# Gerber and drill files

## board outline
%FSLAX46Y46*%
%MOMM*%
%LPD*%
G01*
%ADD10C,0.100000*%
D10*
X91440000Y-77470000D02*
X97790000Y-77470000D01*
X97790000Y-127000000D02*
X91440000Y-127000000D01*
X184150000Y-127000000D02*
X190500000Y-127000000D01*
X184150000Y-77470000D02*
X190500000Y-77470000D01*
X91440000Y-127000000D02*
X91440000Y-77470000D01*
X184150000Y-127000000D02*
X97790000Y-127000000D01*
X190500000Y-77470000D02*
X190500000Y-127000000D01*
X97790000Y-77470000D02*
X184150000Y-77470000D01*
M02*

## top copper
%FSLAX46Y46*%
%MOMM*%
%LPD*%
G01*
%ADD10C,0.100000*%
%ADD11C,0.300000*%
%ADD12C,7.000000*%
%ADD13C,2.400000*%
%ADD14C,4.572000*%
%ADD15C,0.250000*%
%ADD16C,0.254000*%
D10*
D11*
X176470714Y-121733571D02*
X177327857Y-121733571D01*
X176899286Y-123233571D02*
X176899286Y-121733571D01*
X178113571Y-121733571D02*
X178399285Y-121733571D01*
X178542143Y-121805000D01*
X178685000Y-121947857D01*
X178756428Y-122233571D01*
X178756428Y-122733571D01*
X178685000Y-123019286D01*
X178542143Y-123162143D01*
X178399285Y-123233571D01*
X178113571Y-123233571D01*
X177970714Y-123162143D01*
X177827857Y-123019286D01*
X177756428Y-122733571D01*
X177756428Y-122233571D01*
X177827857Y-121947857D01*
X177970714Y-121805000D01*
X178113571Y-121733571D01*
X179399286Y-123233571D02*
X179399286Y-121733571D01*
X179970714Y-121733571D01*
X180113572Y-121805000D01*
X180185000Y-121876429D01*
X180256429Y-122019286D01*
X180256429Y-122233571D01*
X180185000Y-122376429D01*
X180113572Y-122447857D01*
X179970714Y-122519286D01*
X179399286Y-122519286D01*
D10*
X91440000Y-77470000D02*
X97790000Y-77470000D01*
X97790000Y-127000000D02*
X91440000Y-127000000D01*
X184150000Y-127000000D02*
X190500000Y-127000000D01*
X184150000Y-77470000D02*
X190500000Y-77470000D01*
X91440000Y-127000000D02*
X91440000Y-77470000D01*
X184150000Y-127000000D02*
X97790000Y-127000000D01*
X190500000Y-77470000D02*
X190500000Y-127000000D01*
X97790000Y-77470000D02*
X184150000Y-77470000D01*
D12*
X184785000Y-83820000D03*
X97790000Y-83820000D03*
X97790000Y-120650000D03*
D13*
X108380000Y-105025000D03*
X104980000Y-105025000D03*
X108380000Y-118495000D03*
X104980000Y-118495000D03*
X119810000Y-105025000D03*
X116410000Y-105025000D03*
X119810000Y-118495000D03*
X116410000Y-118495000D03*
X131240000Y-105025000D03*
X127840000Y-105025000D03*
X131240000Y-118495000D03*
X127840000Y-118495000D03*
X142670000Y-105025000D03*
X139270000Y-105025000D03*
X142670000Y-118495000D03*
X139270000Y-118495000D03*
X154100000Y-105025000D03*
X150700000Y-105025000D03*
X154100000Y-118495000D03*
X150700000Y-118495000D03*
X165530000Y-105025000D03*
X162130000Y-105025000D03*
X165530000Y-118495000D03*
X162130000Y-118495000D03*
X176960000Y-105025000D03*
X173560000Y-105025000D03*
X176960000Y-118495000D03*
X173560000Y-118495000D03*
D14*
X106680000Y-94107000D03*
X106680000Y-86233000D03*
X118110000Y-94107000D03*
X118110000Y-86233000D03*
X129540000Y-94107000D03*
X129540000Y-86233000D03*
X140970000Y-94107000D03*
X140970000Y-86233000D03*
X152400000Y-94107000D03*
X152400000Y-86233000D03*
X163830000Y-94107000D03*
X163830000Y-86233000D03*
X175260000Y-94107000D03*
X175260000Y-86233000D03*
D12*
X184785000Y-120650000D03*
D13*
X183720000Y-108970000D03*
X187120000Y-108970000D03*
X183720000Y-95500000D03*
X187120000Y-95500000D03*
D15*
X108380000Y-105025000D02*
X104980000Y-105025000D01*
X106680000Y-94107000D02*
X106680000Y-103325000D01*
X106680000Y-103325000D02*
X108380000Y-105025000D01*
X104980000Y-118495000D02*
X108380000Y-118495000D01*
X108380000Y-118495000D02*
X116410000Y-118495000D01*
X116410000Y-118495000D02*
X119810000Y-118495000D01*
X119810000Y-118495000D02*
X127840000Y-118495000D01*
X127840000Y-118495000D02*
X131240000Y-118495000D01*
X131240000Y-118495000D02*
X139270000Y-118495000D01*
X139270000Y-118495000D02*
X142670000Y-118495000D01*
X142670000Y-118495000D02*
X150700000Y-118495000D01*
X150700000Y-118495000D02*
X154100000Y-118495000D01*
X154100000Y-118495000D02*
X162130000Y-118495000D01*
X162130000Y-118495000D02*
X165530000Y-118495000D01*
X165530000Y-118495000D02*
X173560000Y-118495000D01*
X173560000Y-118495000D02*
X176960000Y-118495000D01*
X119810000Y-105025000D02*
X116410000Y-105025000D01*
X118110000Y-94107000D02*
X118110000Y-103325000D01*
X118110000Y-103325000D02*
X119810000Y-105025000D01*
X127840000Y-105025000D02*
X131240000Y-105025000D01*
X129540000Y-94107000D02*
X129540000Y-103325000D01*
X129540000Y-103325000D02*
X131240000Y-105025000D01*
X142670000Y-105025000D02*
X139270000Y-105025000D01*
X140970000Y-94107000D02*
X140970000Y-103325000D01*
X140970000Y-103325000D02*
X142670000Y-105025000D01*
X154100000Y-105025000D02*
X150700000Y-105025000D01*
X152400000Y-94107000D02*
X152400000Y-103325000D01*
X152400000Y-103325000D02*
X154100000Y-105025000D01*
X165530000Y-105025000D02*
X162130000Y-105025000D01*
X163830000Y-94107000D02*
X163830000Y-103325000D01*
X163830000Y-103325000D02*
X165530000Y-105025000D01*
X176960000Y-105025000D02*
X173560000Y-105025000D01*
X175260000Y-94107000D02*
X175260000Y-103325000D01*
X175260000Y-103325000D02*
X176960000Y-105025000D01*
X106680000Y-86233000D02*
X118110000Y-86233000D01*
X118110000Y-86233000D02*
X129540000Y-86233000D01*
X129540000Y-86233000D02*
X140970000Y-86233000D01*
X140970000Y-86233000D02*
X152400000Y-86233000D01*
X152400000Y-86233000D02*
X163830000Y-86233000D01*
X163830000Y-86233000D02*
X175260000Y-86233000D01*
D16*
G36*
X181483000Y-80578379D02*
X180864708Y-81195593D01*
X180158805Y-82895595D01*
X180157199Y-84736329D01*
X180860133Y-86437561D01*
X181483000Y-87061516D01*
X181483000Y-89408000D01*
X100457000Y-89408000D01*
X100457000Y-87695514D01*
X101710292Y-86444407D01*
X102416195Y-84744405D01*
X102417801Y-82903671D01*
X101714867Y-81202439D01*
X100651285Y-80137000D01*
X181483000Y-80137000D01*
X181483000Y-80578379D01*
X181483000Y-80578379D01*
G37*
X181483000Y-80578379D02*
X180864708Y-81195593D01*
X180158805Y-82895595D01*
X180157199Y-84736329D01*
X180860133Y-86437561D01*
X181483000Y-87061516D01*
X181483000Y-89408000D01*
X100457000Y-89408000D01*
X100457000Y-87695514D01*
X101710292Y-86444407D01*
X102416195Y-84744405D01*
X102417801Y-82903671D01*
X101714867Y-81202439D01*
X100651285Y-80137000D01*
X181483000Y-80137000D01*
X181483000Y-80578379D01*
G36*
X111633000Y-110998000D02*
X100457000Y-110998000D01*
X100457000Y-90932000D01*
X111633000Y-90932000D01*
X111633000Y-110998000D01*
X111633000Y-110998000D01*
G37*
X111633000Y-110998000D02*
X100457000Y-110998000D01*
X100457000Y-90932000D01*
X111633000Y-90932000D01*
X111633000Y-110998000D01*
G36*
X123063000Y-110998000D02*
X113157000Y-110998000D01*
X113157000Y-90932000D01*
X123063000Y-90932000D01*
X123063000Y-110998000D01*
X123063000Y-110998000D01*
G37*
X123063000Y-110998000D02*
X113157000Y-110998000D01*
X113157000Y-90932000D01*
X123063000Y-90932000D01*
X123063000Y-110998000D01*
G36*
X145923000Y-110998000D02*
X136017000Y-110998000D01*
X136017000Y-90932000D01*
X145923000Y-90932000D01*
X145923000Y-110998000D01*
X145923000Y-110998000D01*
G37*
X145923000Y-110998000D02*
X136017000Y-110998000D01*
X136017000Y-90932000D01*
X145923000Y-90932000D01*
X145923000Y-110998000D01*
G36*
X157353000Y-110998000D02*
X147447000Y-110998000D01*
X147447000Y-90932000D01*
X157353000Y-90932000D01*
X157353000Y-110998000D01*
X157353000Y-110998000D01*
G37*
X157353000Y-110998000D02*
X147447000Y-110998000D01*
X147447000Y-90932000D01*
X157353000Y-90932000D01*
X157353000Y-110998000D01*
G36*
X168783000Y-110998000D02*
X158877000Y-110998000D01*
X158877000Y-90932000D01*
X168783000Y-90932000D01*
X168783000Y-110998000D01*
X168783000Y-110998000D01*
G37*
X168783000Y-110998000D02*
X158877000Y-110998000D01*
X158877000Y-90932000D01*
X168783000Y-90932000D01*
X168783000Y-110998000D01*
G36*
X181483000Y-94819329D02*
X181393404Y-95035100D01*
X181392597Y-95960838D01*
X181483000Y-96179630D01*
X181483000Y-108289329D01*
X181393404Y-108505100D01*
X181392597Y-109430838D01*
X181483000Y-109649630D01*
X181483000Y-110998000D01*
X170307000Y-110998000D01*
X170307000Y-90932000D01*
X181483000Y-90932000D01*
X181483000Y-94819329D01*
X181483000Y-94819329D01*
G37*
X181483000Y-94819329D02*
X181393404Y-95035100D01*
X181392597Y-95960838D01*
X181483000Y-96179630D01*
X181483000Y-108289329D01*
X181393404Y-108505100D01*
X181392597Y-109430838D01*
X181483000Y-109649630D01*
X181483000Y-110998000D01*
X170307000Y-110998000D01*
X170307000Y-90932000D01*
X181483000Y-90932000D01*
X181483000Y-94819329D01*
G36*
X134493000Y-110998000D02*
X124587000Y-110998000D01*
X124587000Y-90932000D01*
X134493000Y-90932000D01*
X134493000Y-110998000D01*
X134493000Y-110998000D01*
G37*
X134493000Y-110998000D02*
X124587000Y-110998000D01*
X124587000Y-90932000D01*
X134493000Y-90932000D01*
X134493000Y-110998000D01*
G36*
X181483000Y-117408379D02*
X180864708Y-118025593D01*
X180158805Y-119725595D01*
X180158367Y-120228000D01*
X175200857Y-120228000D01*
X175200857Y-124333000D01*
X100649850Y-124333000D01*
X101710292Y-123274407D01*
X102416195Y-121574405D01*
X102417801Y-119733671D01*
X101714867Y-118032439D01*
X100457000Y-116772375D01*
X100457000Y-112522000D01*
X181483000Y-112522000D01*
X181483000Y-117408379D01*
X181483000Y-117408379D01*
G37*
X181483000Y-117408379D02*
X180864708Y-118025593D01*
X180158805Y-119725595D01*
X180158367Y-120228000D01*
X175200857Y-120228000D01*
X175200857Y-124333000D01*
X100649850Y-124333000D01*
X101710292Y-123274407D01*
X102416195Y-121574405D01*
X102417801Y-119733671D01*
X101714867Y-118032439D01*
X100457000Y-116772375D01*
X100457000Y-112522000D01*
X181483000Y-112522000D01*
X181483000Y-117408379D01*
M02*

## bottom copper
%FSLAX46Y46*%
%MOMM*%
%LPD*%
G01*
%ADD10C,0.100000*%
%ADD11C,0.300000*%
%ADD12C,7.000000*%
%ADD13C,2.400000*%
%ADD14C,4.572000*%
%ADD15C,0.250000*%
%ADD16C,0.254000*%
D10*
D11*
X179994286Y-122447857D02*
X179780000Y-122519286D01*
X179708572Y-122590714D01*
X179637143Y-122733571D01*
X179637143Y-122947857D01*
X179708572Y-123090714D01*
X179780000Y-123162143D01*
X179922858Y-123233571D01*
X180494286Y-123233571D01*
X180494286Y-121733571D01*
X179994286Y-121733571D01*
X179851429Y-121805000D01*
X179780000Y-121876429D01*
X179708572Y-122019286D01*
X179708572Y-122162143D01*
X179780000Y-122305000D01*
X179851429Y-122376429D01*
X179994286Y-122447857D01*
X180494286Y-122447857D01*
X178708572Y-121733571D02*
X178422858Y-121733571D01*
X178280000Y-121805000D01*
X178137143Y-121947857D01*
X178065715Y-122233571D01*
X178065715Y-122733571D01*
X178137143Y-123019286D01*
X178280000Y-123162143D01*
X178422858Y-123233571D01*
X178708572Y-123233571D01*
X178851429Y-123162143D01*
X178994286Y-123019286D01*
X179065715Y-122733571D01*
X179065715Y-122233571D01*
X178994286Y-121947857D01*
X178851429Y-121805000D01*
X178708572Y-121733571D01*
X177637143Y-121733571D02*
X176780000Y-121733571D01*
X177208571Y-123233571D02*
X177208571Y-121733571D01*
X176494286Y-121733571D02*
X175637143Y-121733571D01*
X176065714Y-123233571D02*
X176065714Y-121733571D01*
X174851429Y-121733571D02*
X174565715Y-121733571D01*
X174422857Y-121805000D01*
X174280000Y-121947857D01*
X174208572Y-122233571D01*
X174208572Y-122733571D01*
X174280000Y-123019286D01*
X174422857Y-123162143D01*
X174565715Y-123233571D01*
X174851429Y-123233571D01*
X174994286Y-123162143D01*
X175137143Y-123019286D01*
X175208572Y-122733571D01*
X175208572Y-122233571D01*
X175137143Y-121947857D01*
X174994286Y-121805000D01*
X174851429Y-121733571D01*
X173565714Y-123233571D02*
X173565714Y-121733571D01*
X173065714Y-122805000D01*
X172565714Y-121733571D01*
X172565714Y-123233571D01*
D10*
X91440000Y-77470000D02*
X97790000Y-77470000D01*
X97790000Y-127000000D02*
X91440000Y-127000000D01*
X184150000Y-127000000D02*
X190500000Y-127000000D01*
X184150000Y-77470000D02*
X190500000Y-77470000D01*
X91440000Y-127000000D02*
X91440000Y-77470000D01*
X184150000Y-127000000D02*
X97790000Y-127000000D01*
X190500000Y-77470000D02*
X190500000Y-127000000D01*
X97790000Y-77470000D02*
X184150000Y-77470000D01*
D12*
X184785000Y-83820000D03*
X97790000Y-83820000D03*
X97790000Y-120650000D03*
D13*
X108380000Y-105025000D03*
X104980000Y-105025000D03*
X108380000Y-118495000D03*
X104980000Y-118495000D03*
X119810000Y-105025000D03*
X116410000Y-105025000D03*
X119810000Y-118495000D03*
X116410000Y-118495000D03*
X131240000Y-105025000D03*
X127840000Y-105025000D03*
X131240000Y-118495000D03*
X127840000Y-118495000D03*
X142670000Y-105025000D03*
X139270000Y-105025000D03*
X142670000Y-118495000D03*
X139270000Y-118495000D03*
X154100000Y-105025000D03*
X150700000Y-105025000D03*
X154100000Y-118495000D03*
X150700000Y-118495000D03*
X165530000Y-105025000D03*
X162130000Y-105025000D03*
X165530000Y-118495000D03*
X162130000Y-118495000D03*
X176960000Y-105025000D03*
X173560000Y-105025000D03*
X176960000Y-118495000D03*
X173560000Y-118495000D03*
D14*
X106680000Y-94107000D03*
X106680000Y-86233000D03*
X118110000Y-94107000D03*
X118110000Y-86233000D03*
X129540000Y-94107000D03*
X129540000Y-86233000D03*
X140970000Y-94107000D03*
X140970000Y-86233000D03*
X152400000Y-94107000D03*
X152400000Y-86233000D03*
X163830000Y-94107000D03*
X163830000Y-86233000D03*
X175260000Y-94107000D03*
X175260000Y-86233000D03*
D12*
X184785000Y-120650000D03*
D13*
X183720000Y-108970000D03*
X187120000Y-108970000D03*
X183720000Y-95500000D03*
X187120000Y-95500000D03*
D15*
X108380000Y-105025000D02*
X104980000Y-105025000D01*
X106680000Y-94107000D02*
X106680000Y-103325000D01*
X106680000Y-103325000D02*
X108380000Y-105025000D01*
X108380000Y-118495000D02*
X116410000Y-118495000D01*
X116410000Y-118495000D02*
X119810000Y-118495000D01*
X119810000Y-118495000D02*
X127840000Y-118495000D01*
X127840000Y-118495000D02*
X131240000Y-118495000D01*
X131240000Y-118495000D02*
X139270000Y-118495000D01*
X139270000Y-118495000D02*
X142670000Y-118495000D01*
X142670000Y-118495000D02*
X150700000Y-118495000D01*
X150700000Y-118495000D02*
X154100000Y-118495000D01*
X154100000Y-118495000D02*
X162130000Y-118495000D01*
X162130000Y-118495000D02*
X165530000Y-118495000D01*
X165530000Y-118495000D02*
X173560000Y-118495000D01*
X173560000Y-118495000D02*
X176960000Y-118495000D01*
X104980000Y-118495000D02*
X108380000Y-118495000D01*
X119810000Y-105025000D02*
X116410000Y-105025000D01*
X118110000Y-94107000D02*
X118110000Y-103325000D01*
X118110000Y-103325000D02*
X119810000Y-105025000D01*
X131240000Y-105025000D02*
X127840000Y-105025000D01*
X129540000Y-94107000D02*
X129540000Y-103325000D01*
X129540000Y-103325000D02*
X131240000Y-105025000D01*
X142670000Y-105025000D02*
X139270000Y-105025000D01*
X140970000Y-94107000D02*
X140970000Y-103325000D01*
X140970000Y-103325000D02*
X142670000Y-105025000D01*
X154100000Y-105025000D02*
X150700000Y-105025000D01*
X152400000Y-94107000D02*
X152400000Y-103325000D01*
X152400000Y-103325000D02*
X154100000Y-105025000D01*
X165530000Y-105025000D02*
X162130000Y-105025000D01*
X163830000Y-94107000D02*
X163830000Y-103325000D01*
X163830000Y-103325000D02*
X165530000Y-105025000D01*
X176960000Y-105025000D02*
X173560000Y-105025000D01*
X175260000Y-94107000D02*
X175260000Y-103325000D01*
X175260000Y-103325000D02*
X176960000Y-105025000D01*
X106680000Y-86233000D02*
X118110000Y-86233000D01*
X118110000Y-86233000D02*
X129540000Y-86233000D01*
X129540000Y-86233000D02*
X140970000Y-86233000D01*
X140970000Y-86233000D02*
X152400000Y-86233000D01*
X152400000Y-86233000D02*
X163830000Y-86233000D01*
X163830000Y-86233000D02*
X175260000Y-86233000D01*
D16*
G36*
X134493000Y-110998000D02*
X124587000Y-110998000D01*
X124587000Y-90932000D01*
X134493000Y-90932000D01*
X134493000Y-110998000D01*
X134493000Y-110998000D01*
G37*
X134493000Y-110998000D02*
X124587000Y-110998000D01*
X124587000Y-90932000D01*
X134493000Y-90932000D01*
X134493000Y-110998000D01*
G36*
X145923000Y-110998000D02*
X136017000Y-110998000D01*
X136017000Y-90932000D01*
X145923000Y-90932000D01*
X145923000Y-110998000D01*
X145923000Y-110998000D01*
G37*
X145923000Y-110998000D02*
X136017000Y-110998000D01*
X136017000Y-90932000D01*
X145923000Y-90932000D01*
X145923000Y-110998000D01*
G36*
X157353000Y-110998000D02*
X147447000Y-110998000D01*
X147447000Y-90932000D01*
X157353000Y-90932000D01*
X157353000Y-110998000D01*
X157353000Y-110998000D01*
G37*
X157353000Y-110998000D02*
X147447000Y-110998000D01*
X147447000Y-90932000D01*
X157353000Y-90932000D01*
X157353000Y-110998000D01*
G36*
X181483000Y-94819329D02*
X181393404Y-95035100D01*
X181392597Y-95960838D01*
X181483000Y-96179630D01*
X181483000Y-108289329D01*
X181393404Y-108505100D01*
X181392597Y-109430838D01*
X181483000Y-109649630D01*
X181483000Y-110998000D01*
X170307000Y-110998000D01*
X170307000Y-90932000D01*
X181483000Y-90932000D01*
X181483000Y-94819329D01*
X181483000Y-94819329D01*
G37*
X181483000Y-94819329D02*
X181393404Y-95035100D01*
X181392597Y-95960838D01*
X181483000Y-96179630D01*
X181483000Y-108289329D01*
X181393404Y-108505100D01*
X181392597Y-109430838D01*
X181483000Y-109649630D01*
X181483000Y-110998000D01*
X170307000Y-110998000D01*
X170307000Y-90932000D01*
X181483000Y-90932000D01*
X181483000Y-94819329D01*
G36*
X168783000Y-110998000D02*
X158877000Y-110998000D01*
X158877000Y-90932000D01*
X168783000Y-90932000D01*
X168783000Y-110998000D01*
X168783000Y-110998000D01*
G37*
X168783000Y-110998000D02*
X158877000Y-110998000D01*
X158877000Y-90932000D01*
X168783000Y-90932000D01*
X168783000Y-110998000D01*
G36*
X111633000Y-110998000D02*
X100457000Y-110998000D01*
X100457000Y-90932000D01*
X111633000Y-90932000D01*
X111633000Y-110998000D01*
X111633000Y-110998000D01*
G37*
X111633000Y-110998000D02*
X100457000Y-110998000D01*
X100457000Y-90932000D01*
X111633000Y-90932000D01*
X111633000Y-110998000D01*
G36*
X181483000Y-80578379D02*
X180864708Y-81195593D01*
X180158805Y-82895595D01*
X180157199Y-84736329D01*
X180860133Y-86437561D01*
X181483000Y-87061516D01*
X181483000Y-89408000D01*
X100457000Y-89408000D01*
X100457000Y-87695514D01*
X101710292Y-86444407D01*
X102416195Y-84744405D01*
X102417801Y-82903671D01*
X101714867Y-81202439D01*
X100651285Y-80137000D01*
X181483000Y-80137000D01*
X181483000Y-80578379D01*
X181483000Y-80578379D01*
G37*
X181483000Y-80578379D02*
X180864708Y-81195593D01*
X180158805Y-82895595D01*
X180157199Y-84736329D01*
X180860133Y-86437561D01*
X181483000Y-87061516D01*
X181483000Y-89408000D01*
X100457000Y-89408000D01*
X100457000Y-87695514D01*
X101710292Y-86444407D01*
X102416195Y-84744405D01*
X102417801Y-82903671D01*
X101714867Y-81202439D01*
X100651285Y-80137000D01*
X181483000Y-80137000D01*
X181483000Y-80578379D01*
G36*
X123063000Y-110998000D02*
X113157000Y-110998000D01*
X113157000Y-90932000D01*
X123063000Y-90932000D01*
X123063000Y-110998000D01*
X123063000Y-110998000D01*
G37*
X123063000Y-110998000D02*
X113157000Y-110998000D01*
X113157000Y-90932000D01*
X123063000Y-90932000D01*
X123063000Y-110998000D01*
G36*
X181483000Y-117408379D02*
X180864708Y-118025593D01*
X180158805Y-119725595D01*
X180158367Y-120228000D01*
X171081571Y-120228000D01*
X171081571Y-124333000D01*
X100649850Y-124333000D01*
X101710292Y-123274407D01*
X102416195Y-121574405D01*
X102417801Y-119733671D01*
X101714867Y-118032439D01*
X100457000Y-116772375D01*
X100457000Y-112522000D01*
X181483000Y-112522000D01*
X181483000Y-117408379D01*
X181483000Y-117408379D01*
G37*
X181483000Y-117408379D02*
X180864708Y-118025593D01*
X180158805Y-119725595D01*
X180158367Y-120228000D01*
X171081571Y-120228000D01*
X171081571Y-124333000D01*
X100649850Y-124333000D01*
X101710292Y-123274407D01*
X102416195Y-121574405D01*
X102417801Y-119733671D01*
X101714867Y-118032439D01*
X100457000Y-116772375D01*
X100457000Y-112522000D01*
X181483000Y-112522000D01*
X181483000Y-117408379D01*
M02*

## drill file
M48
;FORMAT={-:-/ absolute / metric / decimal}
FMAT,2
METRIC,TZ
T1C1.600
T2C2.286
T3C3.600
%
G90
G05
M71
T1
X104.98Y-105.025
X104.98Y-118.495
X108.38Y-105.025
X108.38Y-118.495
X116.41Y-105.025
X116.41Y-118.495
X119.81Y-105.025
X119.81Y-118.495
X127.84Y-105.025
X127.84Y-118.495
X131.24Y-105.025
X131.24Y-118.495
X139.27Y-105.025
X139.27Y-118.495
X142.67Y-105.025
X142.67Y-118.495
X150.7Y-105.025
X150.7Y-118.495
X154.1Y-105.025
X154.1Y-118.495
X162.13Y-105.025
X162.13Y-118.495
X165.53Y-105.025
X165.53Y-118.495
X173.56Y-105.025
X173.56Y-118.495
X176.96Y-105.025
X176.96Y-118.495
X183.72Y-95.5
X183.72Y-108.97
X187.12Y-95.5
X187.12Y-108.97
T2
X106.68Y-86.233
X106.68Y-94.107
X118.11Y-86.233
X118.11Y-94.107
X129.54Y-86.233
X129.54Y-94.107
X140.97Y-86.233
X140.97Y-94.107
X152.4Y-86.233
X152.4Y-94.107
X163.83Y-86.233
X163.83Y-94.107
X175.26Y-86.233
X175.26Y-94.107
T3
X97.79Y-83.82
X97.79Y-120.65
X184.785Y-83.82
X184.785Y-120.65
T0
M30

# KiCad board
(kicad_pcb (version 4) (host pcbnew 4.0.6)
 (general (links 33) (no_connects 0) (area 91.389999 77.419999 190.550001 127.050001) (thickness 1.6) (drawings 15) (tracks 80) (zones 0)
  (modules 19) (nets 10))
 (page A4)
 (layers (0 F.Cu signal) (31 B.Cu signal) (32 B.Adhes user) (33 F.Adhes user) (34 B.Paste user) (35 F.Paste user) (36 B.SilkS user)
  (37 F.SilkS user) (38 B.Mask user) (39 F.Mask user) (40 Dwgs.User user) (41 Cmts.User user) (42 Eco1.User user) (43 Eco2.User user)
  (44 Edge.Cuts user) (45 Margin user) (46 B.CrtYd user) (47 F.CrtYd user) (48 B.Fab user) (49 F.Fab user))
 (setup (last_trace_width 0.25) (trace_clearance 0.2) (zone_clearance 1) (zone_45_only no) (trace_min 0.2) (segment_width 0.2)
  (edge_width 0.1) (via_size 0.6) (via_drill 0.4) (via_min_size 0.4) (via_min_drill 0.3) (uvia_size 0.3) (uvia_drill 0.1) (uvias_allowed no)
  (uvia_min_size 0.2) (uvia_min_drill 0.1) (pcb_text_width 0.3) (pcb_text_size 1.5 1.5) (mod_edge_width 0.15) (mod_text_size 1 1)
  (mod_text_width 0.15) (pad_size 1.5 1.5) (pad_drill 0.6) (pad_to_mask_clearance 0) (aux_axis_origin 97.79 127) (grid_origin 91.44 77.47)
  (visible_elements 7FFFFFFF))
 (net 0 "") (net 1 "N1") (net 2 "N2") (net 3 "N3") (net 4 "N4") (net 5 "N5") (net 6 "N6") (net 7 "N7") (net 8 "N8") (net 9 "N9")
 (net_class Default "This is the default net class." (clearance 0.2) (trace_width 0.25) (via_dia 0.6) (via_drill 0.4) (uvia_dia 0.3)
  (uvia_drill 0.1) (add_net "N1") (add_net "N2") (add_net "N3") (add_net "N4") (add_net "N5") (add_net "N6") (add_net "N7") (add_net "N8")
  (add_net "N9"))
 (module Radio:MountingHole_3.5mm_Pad (layer F.Cu) (at 184.785 83.82)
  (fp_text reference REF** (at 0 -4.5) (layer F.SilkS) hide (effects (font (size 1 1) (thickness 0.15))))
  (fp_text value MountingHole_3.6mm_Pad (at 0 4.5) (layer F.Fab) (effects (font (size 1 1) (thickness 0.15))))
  (pad 1 thru_hole circle (at 0 0) (size 7 7) (drill 3.6) (layers *.Cu *.Mask)))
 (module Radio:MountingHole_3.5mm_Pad (layer F.Cu) (at 97.79 83.82)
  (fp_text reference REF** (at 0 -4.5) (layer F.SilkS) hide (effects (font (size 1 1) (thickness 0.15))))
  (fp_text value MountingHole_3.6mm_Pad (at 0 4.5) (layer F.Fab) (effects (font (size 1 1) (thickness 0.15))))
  (pad 1 thru_hole circle (at 0 0) (size 7 7) (drill 3.6) (layers *.Cu *.Mask)))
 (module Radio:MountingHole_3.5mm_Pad (layer F.Cu) (at 97.79 120.65)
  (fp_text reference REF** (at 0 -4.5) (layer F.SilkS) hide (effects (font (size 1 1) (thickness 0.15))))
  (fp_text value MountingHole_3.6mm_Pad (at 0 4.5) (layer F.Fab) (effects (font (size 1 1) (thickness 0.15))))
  (pad 1 thru_hole circle (at 0 0) (size 7 7) (drill 3.6) (layers *.Cu *.Mask)))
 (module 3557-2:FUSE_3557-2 (layer F.Cu) (at 106.68 111.76 270)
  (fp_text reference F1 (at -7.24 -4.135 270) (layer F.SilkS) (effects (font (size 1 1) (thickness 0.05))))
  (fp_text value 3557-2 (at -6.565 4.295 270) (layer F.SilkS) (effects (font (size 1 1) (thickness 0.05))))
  (pad 1 thru_hole circle (at -6.735 -1.7 270) (size 2.4 2.4) (drill 1.6) (layers *.Cu *.Mask F.SilkS) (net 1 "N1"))
  (pad 2 thru_hole circle (at -6.735 1.7 270) (size 2.4 2.4) (drill 1.6) (layers *.Cu *.Mask F.SilkS) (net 1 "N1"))
  (pad 3 thru_hole circle (at 6.735 -1.7 270) (size 2.4 2.4) (drill 1.6) (layers *.Cu *.Mask F.SilkS) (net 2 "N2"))
  (pad 4 thru_hole circle (at 6.735 1.7 270) (size 2.4 2.4) (drill 1.6) (layers *.Cu *.Mask F.SilkS) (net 2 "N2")))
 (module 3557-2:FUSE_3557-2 (layer F.Cu) (at 118.11 111.76 270)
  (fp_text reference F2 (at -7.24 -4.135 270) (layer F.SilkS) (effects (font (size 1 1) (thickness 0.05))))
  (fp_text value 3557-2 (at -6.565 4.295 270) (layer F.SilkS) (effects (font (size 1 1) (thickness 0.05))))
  (pad 1 thru_hole circle (at -6.735 -1.7 270) (size 2.4 2.4) (drill 1.6) (layers *.Cu *.Mask F.SilkS) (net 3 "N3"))
  (pad 2 thru_hole circle (at -6.735 1.7 270) (size 2.4 2.4) (drill 1.6) (layers *.Cu *.Mask F.SilkS) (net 3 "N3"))
  (pad 3 thru_hole circle (at 6.735 -1.7 270) (size 2.4 2.4) (drill 1.6) (layers *.Cu *.Mask F.SilkS) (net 2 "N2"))
  (pad 4 thru_hole circle (at 6.735 1.7 270) (size 2.4 2.4) (drill 1.6) (layers *.Cu *.Mask F.SilkS) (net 2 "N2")))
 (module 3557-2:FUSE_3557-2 (layer F.Cu) (at 129.54 111.76 270)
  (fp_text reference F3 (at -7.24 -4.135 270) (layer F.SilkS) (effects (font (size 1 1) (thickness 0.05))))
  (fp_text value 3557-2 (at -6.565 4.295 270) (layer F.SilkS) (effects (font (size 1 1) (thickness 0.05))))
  (pad 1 thru_hole circle (at -6.735 -1.7 270) (size 2.4 2.4) (drill 1.6) (layers *.Cu *.Mask F.SilkS) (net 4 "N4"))
  (pad 2 thru_hole circle (at -6.735 1.7 270) (size 2.4 2.4) (drill 1.6) (layers *.Cu *.Mask F.SilkS) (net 4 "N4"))
  (pad 3 thru_hole circle (at 6.735 -1.7 270) (size 2.4 2.4) (drill 1.6) (layers *.Cu *.Mask F.SilkS) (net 2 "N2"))
  (pad 4 thru_hole circle (at 6.735 1.7 270) (size 2.4 2.4) (drill 1.6) (layers *.Cu *.Mask F.SilkS) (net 2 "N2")))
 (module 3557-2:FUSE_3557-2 (layer F.Cu) (at 140.97 111.76 270)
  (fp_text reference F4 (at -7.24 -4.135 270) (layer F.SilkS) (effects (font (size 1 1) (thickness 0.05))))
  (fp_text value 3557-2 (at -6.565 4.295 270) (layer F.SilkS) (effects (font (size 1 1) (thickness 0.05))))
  (pad 1 thru_hole circle (at -6.735 -1.7 270) (size 2.4 2.4) (drill 1.6) (layers *.Cu *.Mask F.SilkS) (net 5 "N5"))
  (pad 2 thru_hole circle (at -6.735 1.7 270) (size 2.4 2.4) (drill 1.6) (layers *.Cu *.Mask F.SilkS) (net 5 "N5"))
  (pad 3 thru_hole circle (at 6.735 -1.7 270) (size 2.4 2.4) (drill 1.6) (layers *.Cu *.Mask F.SilkS) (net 2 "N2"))
  (pad 4 thru_hole circle (at 6.735 1.7 270) (size 2.4 2.4) (drill 1.6) (layers *.Cu *.Mask F.SilkS) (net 2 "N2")))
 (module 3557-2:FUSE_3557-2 (layer F.Cu) (at 152.4 111.76 270)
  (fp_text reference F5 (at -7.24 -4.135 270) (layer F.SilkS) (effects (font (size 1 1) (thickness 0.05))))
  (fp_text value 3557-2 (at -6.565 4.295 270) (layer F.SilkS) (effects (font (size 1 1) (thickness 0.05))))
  (pad 1 thru_hole circle (at -6.735 -1.7 270) (size 2.4 2.4) (drill 1.6) (layers *.Cu *.Mask F.SilkS) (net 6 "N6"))
  (pad 2 thru_hole circle (at -6.735 1.7 270) (size 2.4 2.4) (drill 1.6) (layers *.Cu *.Mask F.SilkS) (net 6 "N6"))
  (pad 3 thru_hole circle (at 6.735 -1.7 270) (size 2.4 2.4) (drill 1.6) (layers *.Cu *.Mask F.SilkS) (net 2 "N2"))
  (pad 4 thru_hole circle (at 6.735 1.7 270) (size 2.4 2.4) (drill 1.6) (layers *.Cu *.Mask F.SilkS) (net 2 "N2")))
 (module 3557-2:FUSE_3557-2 (layer F.Cu) (at 163.83 111.76 270)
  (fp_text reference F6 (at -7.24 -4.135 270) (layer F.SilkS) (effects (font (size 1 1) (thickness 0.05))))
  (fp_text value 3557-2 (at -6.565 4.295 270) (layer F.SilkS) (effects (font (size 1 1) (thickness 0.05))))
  (pad 1 thru_hole circle (at -6.735 -1.7 270) (size 2.4 2.4) (drill 1.6) (layers *.Cu *.Mask F.SilkS) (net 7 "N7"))
  (pad 2 thru_hole circle (at -6.735 1.7 270) (size 2.4 2.4) (drill 1.6) (layers *.Cu *.Mask F.SilkS) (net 7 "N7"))
  (pad 3 thru_hole circle (at 6.735 -1.7 270) (size 2.4 2.4) (drill 1.6) (layers *.Cu *.Mask F.SilkS) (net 2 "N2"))
  (pad 4 thru_hole circle (at 6.735 1.7 270) (size 2.4 2.4) (drill 1.6) (layers *.Cu *.Mask F.SilkS) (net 2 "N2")))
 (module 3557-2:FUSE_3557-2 (layer F.Cu) (at 175.26 111.76 270)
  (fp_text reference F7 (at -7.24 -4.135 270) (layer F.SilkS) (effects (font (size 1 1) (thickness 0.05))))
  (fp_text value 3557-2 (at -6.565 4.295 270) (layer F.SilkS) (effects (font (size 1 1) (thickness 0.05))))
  (pad 1 thru_hole circle (at -6.735 -1.7 270) (size 2.4 2.4) (drill 1.6) (layers *.Cu *.Mask F.SilkS) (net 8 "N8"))
  (pad 2 thru_hole circle (at -6.735 1.7 270) (size 2.4 2.4) (drill 1.6) (layers *.Cu *.Mask F.SilkS) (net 8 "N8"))
  (pad 3 thru_hole circle (at 6.735 -1.7 270) (size 2.4 2.4) (drill 1.6) (layers *.Cu *.Mask F.SilkS) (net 2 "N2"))
  (pad 4 thru_hole circle (at 6.735 1.7 270) (size 2.4 2.4) (drill 1.6) (layers *.Cu *.Mask F.SilkS) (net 2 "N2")))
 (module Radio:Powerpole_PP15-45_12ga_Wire (layer F.Cu) (at 106.68 90.17 90)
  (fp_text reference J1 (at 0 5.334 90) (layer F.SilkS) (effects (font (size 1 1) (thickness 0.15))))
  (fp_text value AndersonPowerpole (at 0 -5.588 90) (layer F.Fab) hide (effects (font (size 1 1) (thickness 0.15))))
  (pad 1 thru_hole circle (at -3.937 0 90) (size 4.572 4.572) (drill 2.286) (layers *.Cu *.Mask) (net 1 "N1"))
  (pad 2 thru_hole circle (at 3.937 0 90) (size 4.572 4.572) (drill 2.286) (layers *.Cu *.Mask) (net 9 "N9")))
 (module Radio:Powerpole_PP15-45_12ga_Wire (layer F.Cu) (at 118.11 90.17 90)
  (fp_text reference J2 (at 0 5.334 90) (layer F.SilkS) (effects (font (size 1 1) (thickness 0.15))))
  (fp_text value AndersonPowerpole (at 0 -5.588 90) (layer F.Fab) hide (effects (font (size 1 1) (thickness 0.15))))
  (pad 1 thru_hole circle (at -3.937 0 90) (size 4.572 4.572) (drill 2.286) (layers *.Cu *.Mask) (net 3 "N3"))
  (pad 2 thru_hole circle (at 3.937 0 90) (size 4.572 4.572) (drill 2.286) (layers *.Cu *.Mask) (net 9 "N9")))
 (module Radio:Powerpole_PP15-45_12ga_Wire (layer F.Cu) (at 129.54 90.17 90)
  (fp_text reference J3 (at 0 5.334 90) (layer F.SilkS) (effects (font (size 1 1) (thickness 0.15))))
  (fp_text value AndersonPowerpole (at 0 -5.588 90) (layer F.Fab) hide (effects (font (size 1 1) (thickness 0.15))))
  (pad 1 thru_hole circle (at -3.937 0 90) (size 4.572 4.572) (drill 2.286) (layers *.Cu *.Mask) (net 4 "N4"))
  (pad 2 thru_hole circle (at 3.937 0 90) (size 4.572 4.572) (drill 2.286) (layers *.Cu *.Mask) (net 9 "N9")))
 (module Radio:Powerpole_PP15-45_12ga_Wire (layer F.Cu) (at 140.97 90.17 90)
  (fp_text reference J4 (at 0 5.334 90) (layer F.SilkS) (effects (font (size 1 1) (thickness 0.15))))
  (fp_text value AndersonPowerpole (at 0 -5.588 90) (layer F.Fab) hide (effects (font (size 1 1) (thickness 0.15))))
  (pad 1 thru_hole circle (at -3.937 0 90) (size 4.572 4.572) (drill 2.286) (layers *.Cu *.Mask) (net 5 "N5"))
  (pad 2 thru_hole circle (at 3.937 0 90) (size 4.572 4.572) (drill 2.286) (layers *.Cu *.Mask) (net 9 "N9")))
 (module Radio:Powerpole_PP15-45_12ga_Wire (layer F.Cu) (at 152.4 90.17 90)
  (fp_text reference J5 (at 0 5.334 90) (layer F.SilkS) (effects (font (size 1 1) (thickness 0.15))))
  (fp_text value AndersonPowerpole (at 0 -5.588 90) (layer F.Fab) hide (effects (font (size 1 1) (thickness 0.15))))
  (pad 1 thru_hole circle (at -3.937 0 90) (size 4.572 4.572) (drill 2.286) (layers *.Cu *.Mask) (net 6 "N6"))
  (pad 2 thru_hole circle (at 3.937 0 90) (size 4.572 4.572) (drill 2.286) (layers *.Cu *.Mask) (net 9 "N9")))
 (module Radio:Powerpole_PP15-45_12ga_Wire (layer F.Cu) (at 163.83 90.17 90)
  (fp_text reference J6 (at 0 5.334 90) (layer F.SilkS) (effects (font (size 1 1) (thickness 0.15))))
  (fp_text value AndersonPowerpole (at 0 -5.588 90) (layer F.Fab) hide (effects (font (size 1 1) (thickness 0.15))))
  (pad 1 thru_hole circle (at -3.937 0 90) (size 4.572 4.572) (drill 2.286) (layers *.Cu *.Mask) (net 7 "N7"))
  (pad 2 thru_hole circle (at 3.937 0 90) (size 4.572 4.572) (drill 2.286) (layers *.Cu *.Mask) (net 9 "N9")))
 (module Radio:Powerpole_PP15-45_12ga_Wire (layer F.Cu) (at 175.26 90.17 90)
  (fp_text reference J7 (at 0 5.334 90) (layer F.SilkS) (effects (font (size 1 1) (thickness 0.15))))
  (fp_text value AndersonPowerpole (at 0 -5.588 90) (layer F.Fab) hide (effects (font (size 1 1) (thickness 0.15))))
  (pad 1 thru_hole circle (at -3.937 0 90) (size 4.572 4.572) (drill 2.286) (layers *.Cu *.Mask) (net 8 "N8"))
  (pad 2 thru_hole circle (at 3.937 0 90) (size 4.572 4.572) (drill 2.286) (layers *.Cu *.Mask) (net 9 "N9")))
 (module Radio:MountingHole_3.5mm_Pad (layer F.Cu) (at 184.785 120.65)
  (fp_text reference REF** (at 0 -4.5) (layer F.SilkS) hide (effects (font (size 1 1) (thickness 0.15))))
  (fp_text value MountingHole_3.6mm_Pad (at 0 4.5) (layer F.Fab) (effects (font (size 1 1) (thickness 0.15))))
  (pad 1 thru_hole circle (at 0 0) (size 7 7) (drill 3.6) (layers *.Cu *.Mask)))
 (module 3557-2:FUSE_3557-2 (layer F.Cu) (at 185.42 102.235 90)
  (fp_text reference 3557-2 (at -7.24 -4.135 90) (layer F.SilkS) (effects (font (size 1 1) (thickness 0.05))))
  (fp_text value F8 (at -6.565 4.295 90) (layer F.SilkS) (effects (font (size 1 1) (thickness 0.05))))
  (pad 1 thru_hole circle (at -6.735 -1.7 90) (size 2.4 2.4) (drill 1.6) (layers *.Cu *.Mask F.SilkS))
  (pad 2 thru_hole circle (at -6.735 1.7 90) (size 2.4 2.4) (drill 1.6) (layers *.Cu *.Mask F.SilkS))
  (pad 3 thru_hole circle (at 6.735 -1.7 90) (size 2.4 2.4) (drill 1.6) (layers *.Cu *.Mask F.SilkS))
  (pad 4 thru_hole circle (at 6.735 1.7 90) (size 2.4 2.4) (drill 1.6) (layers *.Cu *.Mask F.SilkS)))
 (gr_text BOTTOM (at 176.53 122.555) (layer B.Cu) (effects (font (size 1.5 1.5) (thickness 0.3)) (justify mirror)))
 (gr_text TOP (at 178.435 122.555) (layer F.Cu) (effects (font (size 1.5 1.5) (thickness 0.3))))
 (gr_line (start 91.44 77.47) (end 97.79 77.47) (angle 90) (layer Edge.Cuts) (width 0.1))
 (gr_line (start 97.79 127) (end 91.44 127) (angle 90) (layer Edge.Cuts) (width 0.1))
 (gr_line (start 184.15 127) (end 190.5 127) (angle 90) (layer Edge.Cuts) (width 0.1))
 (gr_line (start 184.15 77.47) (end 190.5 77.47) (angle 90) (layer Edge.Cuts) (width 0.1))
 (gr_line (start 91.44 127) (end 91.44 77.47) (angle 90) (layer Edge.Cuts) (width 0.1))
 (gr_line (start 184.15 127) (end 97.79 127) (angle 90) (layer Edge.Cuts) (width 0.1))
 (gr_line (start 190.5 77.47) (end 190.5 127) (angle 90) (layer Edge.Cuts) (width 0.1))
 (gr_line (start 97.79 77.47) (end 184.15 77.47) (angle 90) (layer Edge.Cuts) (width 0.1))
 (segment (start 108.38 105.025) (end 104.98 105.025) (width 0.25) (layer B.Cu) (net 1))
 (segment (start 106.68 94.107) (end 106.68 103.325) (width 0.25) (layer B.Cu) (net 1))
 (segment (start 106.68 103.325) (end 108.38 105.025) (width 0.25) (layer B.Cu) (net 1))
 (segment (start 108.38 105.025) (end 104.98 105.025) (width 0.25) (layer F.Cu) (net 1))
 (segment (start 106.68 94.107) (end 106.68 103.325) (width 0.25) (layer F.Cu) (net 1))
 (segment (start 106.68 103.325) (end 108.38 105.025) (width 0.25) (layer F.Cu) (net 1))
 (segment (start 108.38 118.495) (end 116.41 118.495) (width 0.25) (layer B.Cu) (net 2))
 (segment (start 116.41 118.495) (end 119.81 118.495) (width 0.25) (layer B.Cu) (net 2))
 (segment (start 119.81 118.495) (end 127.84 118.495) (width 0.25) (layer B.Cu) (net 2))
 (segment (start 127.84 118.495) (end 131.24 118.495) (width 0.25) (layer B.Cu) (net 2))
 (segment (start 131.24 118.495) (end 139.27 118.495) (width 0.25) (layer B.Cu) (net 2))
 (segment (start 139.27 118.495) (end 142.67 118.495) (width 0.25) (layer B.Cu) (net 2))
 (segment (start 142.67 118.495) (end 150.7 118.495) (width 0.25) (layer B.Cu) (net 2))
 (segment (start 150.7 118.495) (end 154.1 118.495) (width 0.25) (layer B.Cu) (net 2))
 (segment (start 154.1 118.495) (end 162.13 118.495) (width 0.25) (layer B.Cu) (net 2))
 (segment (start 162.13 118.495) (end 165.53 118.495) (width 0.25) (layer B.Cu) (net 2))
 (segment (start 165.53 118.495) (end 173.56 118.495) (width 0.25) (layer B.Cu) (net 2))
 (segment (start 173.56 118.495) (end 176.96 118.495) (width 0.25) (layer B.Cu) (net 2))
 (segment (start 104.98 118.495) (end 108.38 118.495) (width 0.25) (layer B.Cu) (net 2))
 (segment (start 104.98 118.495) (end 108.38 118.495) (width 0.25) (layer F.Cu) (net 2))
 (segment (start 108.38 118.495) (end 116.41 118.495) (width 0.25) (layer F.Cu) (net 2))
 (segment (start 116.41 118.495) (end 119.81 118.495) (width 0.25) (layer F.Cu) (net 2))
 (segment (start 119.81 118.495) (end 127.84 118.495) (width 0.25) (layer F.Cu) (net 2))
 (segment (start 127.84 118.495) (end 131.24 118.495) (width 0.25) (layer F.Cu) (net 2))
 (segment (start 131.24 118.495) (end 139.27 118.495) (width 0.25) (layer F.Cu) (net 2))
 (segment (start 139.27 118.495) (end 142.67 118.495) (width 0.25) (layer F.Cu) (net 2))
 (segment (start 142.67 118.495) (end 150.7 118.495) (width 0.25) (layer F.Cu) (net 2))
 (segment (start 150.7 118.495) (end 154.1 118.495) (width 0.25) (layer F.Cu) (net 2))
 (segment (start 154.1 118.495) (end 162.13 118.495) (width 0.25) (layer F.Cu) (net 2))
 (segment (start 162.13 118.495) (end 165.53 118.495) (width 0.25) (layer F.Cu) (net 2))
 (segment (start 165.53 118.495) (end 173.56 118.495) (width 0.25) (layer F.Cu) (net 2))
 (segment (start 173.56 118.495) (end 176.96 118.495) (width 0.25) (layer F.Cu) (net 2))
 (segment (start 119.81 105.025) (end 116.41 105.025) (width 0.25) (layer B.Cu) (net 3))
 (segment (start 118.11 94.107) (end 118.11 103.325) (width 0.25) (layer B.Cu) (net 3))
 (segment (start 118.11 103.325) (end 119.81 105.025) (width 0.25) (layer B.Cu) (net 3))
 (segment (start 119.81 105.025) (end 116.41 105.025) (width 0.25) (layer F.Cu) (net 3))
 (segment (start 118.11 94.107) (end 118.11 103.325) (width 0.25) (layer F.Cu) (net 3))
 (segment (start 118.11 103.325) (end 119.81 105.025) (width 0.25) (layer F.Cu) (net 3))
 (segment (start 131.24 105.025) (end 127.84 105.025) (width 0.25) (layer B.Cu) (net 4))
 (segment (start 129.54 94.107) (end 129.54 103.325) (width 0.25) (layer B.Cu) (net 4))
 (segment (start 129.54 103.325) (end 131.24 105.025) (width 0.25) (layer B.Cu) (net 4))
 (segment (start 127.84 105.025) (end 131.24 105.025) (width 0.25) (layer F.Cu) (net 4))
 (segment (start 129.54 94.107) (end 129.54 103.325) (width 0.25) (layer F.Cu) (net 4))
 (segment (start 129.54 103.325) (end 131.24 105.025) (width 0.25) (layer F.Cu) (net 4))
 (segment (start 142.67 105.025) (end 139.27 105.025) (width 0.25) (layer B.Cu) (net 5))
 (segment (start 140.97 94.107) (end 140.97 103.325) (width 0.25) (layer B.Cu) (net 5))
 (segment (start 140.97 103.325) (end 142.67 105.025) (width 0.25) (layer B.Cu) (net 5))
 (segment (start 142.67 105.025) (end 139.27 105.025) (width 0.25) (layer F.Cu) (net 5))
 (segment (start 140.97 94.107) (end 140.97 103.325) (width 0.25) (layer F.Cu) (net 5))
 (segment (start 140.97 103.325) (end 142.67 105.025) (width 0.25) (layer F.Cu) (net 5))
 (segment (start 154.1 105.025) (end 150.7 105.025) (width 0.25) (layer B.Cu) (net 6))
 (segment (start 152.4 94.107) (end 152.4 103.325) (width 0.25) (layer B.Cu) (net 6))
 (segment (start 152.4 103.325) (end 154.1 105.025) (width 0.25) (layer B.Cu) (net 6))
 (segment (start 154.1 105.025) (end 150.7 105.025) (width 0.25) (layer F.Cu) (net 6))
 (segment (start 152.4 94.107) (end 152.4 103.325) (width 0.25) (layer F.Cu) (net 6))
 (segment (start 152.4 103.325) (end 154.1 105.025) (width 0.25) (layer F.Cu) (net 6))
 (segment (start 165.53 105.025) (end 162.13 105.025) (width 0.25) (layer B.Cu) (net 7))
 (segment (start 163.83 94.107) (end 163.83 103.325) (width 0.25) (layer B.Cu) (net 7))
 (segment (start 163.83 103.325) (end 165.53 105.025) (width 0.25) (layer B.Cu) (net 7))
 (segment (start 165.53 105.025) (end 162.13 105.025) (width 0.25) (layer F.Cu) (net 7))
 (segment (start 163.83 94.107) (end 163.83 103.325) (width 0.25) (layer F.Cu) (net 7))
 (segment (start 163.83 103.325) (end 165.53 105.025) (width 0.25) (layer F.Cu) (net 7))
 (segment (start 176.96 105.025) (end 173.56 105.025) (width 0.25) (layer B.Cu) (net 8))
 (segment (start 175.26 94.107) (end 175.26 103.325) (width 0.25) (layer B.Cu) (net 8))
 (segment (start 175.26 103.325) (end 176.96 105.025) (width 0.25) (layer B.Cu) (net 8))
 (segment (start 176.96 105.025) (end 173.56 105.025) (width 0.25) (layer F.Cu) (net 8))
 (segment (start 175.26 94.107) (end 175.26 103.325) (width 0.25) (layer F.Cu) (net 8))
 (segment (start 175.26 103.325) (end 176.96 105.025) (width 0.25) (layer F.Cu) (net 8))
 (segment (start 106.68 86.233) (end 118.11 86.233) (width 0.25) (layer B.Cu) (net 9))
 (segment (start 118.11 86.233) (end 129.54 86.233) (width 0.25) (layer B.Cu) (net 9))
 (segment (start 129.54 86.233) (end 140.97 86.233) (width 0.25) (layer B.Cu) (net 9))
 (segment (start 140.97 86.233) (end 152.4 86.233) (width 0.25) (layer B.Cu) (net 9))
 (segment (start 152.4 86.233) (end 163.83 86.233) (width 0.25) (layer B.Cu) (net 9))
 (segment (start 163.83 86.233) (end 175.26 86.233) (width 0.25) (layer B.Cu) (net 9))
 (segment (start 106.68 86.233) (end 118.11 86.233) (width 0.25) (layer F.Cu) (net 9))
 (segment (start 118.11 86.233) (end 129.54 86.233) (width 0.25) (layer F.Cu) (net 9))
 (segment (start 129.54 86.233) (end 140.97 86.233) (width 0.25) (layer F.Cu) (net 9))
 (segment (start 140.97 86.233) (end 152.4 86.233) (width 0.25) (layer F.Cu) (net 9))
 (segment (start 152.4 86.233) (end 163.83 86.233) (width 0.25) (layer F.Cu) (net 9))
 (segment (start 163.83 86.233) (end 175.26 86.233) (width 0.25) (layer F.Cu) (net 9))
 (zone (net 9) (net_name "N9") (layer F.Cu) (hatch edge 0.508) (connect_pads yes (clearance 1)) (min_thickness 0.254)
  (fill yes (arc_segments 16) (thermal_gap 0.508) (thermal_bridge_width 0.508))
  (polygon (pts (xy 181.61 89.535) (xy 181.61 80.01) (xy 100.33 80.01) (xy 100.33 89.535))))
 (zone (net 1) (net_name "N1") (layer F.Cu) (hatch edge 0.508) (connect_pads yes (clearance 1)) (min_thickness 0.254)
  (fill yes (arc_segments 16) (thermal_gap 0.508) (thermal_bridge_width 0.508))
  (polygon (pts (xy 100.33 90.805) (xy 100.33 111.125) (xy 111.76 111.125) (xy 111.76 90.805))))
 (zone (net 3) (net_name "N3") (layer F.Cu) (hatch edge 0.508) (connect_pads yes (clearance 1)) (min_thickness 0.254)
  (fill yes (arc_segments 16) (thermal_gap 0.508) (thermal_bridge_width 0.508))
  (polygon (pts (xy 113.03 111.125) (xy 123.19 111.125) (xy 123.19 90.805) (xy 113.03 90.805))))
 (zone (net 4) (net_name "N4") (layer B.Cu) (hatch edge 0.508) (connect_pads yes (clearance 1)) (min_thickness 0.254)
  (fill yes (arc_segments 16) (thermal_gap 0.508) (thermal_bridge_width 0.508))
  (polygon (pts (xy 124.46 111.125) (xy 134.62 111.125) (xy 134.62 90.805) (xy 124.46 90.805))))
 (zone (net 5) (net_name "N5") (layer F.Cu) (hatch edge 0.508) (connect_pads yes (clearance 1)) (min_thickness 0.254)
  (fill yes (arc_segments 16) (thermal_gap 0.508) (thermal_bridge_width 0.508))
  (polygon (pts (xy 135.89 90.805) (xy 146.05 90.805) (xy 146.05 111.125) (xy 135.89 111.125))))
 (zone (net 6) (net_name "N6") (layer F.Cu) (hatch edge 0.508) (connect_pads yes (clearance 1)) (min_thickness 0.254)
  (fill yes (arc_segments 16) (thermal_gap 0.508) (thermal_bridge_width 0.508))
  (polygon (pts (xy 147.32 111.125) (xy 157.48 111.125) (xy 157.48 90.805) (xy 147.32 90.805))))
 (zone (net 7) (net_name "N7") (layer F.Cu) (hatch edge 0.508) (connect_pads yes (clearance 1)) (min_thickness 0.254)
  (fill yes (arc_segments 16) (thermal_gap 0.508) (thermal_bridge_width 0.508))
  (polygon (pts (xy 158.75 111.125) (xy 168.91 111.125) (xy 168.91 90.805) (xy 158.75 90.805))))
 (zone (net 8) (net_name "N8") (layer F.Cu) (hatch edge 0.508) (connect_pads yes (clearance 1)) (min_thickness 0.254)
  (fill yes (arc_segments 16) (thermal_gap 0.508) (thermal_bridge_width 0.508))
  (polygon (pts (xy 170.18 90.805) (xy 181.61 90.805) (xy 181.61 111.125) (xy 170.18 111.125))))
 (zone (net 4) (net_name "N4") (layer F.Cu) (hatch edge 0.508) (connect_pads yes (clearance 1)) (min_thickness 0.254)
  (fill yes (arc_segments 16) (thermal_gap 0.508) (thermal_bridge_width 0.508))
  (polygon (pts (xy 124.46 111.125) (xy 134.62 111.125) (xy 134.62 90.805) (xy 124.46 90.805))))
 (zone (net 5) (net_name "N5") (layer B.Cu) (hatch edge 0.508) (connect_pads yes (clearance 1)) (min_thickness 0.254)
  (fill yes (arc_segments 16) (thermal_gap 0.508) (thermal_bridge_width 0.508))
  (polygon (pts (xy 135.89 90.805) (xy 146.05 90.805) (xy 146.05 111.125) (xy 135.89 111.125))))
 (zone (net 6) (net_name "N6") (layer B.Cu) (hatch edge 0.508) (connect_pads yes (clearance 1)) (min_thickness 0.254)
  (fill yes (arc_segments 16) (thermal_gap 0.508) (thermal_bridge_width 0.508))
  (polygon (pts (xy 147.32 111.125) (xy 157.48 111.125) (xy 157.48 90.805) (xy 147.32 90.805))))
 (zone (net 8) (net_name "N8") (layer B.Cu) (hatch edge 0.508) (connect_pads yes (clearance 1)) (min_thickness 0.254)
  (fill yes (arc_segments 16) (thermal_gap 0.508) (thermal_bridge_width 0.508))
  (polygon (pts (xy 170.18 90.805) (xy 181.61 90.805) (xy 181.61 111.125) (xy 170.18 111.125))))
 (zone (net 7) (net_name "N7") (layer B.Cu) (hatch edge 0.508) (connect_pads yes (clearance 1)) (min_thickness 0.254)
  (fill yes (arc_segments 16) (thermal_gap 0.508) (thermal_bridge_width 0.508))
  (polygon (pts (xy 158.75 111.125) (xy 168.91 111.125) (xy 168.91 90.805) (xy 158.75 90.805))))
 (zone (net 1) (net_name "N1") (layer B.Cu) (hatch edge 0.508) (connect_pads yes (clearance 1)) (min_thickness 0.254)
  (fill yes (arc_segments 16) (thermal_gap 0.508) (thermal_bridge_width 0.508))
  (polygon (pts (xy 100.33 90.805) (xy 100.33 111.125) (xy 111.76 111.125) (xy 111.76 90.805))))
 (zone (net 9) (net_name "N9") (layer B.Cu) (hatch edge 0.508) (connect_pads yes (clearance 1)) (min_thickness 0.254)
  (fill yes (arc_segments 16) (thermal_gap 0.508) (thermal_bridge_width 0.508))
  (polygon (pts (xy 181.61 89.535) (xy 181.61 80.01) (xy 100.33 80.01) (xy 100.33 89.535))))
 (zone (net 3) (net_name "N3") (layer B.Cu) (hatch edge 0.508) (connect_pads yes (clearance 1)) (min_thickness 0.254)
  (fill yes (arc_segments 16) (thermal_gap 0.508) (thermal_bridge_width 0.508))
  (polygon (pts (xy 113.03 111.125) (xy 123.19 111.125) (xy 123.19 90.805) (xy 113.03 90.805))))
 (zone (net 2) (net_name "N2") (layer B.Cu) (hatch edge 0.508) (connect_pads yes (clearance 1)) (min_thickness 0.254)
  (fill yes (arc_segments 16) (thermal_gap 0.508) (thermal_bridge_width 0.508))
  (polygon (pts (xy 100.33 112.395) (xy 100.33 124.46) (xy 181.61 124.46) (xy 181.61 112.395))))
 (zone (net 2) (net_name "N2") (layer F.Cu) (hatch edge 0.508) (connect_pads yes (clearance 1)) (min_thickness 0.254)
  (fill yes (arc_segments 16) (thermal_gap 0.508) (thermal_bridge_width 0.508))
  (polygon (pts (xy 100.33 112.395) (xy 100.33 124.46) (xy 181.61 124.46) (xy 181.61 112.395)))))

